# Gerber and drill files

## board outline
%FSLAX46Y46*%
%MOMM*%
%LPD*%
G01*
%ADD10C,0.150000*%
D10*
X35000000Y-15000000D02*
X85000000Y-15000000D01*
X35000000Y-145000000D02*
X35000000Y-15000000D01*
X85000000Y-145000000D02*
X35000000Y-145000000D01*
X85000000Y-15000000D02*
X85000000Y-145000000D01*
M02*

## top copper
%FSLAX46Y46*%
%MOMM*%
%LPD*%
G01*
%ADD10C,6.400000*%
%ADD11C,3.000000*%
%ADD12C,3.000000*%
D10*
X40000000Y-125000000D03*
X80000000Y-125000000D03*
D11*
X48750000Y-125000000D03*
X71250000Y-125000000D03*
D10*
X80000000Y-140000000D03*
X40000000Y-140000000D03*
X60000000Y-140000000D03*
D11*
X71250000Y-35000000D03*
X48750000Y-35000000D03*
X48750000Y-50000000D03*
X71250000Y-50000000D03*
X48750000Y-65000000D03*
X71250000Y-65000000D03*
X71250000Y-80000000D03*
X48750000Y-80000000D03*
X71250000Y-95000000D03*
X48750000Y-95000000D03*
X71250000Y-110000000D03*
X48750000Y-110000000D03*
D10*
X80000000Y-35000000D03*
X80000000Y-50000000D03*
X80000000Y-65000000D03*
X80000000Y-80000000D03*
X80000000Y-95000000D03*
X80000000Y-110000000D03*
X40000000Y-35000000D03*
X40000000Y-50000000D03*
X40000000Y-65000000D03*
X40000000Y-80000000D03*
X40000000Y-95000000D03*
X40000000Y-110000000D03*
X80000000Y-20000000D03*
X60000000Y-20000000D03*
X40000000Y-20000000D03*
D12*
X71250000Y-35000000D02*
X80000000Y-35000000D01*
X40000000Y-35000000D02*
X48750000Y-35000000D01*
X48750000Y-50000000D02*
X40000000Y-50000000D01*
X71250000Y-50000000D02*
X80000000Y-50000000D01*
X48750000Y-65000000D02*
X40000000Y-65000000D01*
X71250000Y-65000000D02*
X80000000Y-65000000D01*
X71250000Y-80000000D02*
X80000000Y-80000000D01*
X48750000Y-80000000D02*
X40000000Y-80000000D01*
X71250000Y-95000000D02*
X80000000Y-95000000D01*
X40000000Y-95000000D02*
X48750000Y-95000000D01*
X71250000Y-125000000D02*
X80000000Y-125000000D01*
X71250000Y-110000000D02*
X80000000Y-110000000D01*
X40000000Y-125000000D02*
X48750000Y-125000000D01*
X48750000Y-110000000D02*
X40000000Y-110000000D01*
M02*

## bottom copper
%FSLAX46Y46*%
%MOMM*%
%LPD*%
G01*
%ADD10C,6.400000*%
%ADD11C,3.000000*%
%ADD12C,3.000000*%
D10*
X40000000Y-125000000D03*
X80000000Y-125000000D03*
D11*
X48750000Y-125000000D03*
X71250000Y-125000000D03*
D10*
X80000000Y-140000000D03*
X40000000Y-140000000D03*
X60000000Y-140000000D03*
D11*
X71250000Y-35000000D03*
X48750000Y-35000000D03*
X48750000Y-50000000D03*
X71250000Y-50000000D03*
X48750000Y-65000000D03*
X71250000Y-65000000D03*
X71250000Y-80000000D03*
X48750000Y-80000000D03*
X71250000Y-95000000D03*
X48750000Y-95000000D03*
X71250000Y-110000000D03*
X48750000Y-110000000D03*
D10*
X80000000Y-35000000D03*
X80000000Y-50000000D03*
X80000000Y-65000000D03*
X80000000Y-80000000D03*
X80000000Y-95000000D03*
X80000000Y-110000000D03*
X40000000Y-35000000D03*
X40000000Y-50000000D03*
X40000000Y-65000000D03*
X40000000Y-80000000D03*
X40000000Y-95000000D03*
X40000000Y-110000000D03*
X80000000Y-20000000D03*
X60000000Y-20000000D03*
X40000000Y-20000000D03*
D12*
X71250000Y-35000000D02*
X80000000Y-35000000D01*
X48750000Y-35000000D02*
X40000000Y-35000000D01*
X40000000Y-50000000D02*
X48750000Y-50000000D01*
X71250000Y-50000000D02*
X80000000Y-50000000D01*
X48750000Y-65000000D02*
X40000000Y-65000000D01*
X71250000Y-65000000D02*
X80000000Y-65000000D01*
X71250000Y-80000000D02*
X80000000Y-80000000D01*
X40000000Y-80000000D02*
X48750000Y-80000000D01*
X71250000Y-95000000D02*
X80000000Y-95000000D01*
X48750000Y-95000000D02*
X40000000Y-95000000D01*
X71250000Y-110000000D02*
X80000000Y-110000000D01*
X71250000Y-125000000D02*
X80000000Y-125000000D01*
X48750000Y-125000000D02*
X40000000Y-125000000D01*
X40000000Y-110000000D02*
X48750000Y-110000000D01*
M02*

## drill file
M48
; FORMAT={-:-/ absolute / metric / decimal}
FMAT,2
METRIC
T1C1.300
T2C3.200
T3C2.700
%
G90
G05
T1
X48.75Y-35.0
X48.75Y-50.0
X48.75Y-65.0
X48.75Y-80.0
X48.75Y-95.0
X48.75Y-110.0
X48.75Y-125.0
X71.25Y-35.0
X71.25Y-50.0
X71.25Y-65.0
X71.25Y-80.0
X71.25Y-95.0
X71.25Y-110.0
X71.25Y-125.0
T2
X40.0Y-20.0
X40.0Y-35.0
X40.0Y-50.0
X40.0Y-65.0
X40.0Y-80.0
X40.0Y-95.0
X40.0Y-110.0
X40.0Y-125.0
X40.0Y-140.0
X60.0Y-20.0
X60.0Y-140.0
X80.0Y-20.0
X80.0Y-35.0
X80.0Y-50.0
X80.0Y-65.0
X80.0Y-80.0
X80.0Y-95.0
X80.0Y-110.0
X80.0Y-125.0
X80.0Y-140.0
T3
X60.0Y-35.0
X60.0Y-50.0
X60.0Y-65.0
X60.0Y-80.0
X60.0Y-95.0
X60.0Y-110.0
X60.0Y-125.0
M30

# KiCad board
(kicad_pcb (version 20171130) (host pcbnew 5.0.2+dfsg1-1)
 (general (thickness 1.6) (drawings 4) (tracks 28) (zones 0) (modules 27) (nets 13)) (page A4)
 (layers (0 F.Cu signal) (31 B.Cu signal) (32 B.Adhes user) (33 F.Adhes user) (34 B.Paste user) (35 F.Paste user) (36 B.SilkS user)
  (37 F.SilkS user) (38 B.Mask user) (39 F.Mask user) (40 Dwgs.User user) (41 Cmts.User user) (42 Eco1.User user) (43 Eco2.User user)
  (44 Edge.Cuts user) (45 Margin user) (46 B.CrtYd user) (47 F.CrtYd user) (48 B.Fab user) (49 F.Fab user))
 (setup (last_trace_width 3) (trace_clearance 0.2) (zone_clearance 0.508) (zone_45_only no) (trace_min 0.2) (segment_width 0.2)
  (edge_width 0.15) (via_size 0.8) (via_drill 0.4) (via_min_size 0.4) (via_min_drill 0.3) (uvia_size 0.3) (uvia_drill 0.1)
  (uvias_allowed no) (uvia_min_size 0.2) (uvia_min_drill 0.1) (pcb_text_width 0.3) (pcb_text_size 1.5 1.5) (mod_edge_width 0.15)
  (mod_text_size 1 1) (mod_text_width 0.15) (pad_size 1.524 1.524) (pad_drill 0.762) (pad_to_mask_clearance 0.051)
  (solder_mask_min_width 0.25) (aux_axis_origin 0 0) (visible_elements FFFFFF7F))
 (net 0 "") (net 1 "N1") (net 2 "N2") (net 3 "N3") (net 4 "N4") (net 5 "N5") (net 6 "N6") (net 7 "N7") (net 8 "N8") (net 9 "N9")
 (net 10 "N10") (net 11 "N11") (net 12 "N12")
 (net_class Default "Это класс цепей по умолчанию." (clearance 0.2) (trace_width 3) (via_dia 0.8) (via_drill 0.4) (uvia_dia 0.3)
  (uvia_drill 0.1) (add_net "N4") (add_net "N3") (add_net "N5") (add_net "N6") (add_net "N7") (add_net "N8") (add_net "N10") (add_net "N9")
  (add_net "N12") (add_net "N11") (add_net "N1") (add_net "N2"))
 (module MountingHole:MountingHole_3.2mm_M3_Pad (layer F.Cu) (at 40 125)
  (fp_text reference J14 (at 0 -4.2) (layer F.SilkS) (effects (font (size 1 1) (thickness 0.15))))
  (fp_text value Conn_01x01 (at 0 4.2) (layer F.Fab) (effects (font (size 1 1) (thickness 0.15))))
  (pad 1 thru_hole circle (at 0 0) (size 6.4 6.4) (drill 3.2) (layers *.Cu *.Mask) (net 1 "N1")))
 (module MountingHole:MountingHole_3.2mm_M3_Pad (layer F.Cu) (at 80 125)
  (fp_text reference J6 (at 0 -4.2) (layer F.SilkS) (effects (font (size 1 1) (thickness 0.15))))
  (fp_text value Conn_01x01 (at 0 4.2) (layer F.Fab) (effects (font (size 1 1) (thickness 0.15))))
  (pad 1 thru_hole circle (at 0 0) (size 6.4 6.4) (drill 3.2) (layers *.Cu *.Mask) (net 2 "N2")))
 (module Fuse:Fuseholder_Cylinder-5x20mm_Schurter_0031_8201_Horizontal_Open (layer F.Cu) (at 48.75 125)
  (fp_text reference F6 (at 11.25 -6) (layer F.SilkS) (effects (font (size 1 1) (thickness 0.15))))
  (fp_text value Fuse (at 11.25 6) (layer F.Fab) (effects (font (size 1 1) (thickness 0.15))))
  (pad 1 thru_hole circle (at 0 0) (size 3 3) (drill 1.3) (layers *.Cu *.Mask) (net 1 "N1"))
  (pad 2 thru_hole circle (at 22.5 0) (size 3 3) (drill 1.3) (layers *.Cu *.Mask) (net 2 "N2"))
  (pad "" np_thru_hole circle (at 11.25 0) (size 2.7 2.7) (drill 2.7) (layers *.Cu *.Mask)))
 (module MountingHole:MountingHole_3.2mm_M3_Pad (layer F.Cu) (at 80 140)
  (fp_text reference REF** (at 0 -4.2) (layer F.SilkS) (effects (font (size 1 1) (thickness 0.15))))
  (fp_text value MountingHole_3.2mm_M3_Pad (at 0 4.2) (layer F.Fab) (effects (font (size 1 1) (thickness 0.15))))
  (pad 1 thru_hole circle (at 0 0) (size 6.4 6.4) (drill 3.2) (layers *.Cu *.Mask)))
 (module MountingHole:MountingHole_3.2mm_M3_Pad (layer F.Cu) (at 40 140)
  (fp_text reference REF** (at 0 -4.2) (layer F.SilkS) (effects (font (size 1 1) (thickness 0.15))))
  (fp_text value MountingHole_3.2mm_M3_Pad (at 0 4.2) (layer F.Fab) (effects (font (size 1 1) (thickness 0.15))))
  (pad 1 thru_hole circle (at 0 0) (size 6.4 6.4) (drill 3.2) (layers *.Cu *.Mask)))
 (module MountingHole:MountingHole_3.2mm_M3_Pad (layer F.Cu) (at 60 140)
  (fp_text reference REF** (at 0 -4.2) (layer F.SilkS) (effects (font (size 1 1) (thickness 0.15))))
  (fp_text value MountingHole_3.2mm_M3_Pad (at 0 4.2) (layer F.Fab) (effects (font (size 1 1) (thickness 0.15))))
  (pad 1 thru_hole circle (at 0 0) (size 6.4 6.4) (drill 3.2) (layers *.Cu *.Mask)))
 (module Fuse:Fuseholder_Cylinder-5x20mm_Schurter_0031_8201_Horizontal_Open (layer F.Cu) (at 48.75 35)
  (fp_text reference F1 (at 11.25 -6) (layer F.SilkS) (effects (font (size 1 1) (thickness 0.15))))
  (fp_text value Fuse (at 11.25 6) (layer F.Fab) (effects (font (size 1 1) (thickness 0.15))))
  (pad "" np_thru_hole circle (at 11.25 0) (size 2.7 2.7) (drill 2.7) (layers *.Cu *.Mask))
  (pad 2 thru_hole circle (at 22.5 0) (size 3 3) (drill 1.3) (layers *.Cu *.Mask) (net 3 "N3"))
  (pad 1 thru_hole circle (at 0 0) (size 3 3) (drill 1.3) (layers *.Cu *.Mask) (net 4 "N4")))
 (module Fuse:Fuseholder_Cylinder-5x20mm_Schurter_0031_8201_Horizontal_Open (layer F.Cu) (at 48.75 50)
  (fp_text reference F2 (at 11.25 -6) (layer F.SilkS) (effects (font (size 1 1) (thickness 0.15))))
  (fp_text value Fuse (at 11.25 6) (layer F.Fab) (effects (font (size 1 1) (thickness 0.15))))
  (pad 1 thru_hole circle (at 0 0) (size 3 3) (drill 1.3) (layers *.Cu *.Mask) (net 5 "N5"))
  (pad 2 thru_hole circle (at 22.5 0) (size 3 3) (drill 1.3) (layers *.Cu *.Mask) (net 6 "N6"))
  (pad "" np_thru_hole circle (at 11.25 0) (size 2.7 2.7) (drill 2.7) (layers *.Cu *.Mask)))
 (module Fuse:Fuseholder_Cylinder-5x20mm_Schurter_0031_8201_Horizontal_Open (layer F.Cu) (at 48.75 65)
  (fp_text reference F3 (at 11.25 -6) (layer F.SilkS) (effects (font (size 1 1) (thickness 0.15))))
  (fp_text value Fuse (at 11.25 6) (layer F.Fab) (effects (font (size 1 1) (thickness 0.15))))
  (pad 1 thru_hole circle (at 0 0) (size 3 3) (drill 1.3) (layers *.Cu *.Mask) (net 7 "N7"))
  (pad 2 thru_hole circle (at 22.5 0) (size 3 3) (drill 1.3) (layers *.Cu *.Mask) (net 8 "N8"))
  (pad "" np_thru_hole circle (at 11.25 0) (size 2.7 2.7) (drill 2.7) (layers *.Cu *.Mask)))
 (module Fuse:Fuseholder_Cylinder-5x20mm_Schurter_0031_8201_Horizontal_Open (layer F.Cu) (at 48.75 80)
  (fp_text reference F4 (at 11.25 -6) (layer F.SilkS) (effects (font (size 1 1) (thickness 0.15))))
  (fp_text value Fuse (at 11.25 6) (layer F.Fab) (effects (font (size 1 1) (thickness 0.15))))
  (pad "" np_thru_hole circle (at 11.25 0) (size 2.7 2.7) (drill 2.7) (layers *.Cu *.Mask))
  (pad 2 thru_hole circle (at 22.5 0) (size 3 3) (drill 1.3) (layers *.Cu *.Mask) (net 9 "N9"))
  (pad 1 thru_hole circle (at 0 0) (size 3 3) (drill 1.3) (layers *.Cu *.Mask) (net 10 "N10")))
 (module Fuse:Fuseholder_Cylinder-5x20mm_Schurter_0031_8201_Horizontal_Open (layer F.Cu) (at 48.75 95)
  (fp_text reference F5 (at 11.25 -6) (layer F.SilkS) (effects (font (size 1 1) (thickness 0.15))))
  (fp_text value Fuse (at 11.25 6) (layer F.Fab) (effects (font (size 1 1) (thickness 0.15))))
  (pad "" np_thru_hole circle (at 11.25 0) (size 2.7 2.7) (drill 2.7) (layers *.Cu *.Mask))
  (pad 2 thru_hole circle (at 22.5 0) (size 3 3) (drill 1.3) (layers *.Cu *.Mask) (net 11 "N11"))
  (pad 1 thru_hole circle (at 0 0) (size 3 3) (drill 1.3) (layers *.Cu *.Mask) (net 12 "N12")))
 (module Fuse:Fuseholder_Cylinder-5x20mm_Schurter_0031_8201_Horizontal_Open (layer F.Cu) (at 48.75 110)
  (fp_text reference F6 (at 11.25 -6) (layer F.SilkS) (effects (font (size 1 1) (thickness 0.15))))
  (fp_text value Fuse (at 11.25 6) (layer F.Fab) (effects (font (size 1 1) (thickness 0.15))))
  (pad "" np_thru_hole circle (at 11.25 0) (size 2.7 2.7) (drill 2.7) (layers *.Cu *.Mask))
  (pad 2 thru_hole circle (at 22.5 0) (size 3 3) (drill 1.3) (layers *.Cu *.Mask) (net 2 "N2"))
  (pad 1 thru_hole circle (at 0 0) (size 3 3) (drill 1.3) (layers *.Cu *.Mask) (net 1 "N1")))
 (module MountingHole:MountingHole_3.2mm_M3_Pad (layer F.Cu) (at 80 35)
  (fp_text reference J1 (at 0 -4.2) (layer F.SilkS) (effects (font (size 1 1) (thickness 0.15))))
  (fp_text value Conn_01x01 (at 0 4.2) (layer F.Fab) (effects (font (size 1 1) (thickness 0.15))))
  (pad 1 thru_hole circle (at 0 0) (size 6.4 6.4) (drill 3.2) (layers *.Cu *.Mask) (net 3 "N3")))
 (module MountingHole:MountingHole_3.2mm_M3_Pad (layer F.Cu) (at 80 50)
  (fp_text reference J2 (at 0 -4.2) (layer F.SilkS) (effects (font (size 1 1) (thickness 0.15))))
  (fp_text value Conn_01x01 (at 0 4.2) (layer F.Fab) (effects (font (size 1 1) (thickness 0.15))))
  (pad 1 thru_hole circle (at 0 0) (size 6.4 6.4) (drill 3.2) (layers *.Cu *.Mask) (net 6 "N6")))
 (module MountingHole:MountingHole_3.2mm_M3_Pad (layer F.Cu) (at 80 65)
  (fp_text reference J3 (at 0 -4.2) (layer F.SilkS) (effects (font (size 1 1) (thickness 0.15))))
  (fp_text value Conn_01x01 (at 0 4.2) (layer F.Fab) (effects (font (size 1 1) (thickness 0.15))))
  (pad 1 thru_hole circle (at 0 0) (size 6.4 6.4) (drill 3.2) (layers *.Cu *.Mask) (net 8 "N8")))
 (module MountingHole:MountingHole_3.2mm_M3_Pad (layer F.Cu) (at 80 80)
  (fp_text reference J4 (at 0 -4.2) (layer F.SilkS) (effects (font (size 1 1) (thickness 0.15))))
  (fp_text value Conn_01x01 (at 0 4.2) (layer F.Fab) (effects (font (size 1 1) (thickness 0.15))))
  (pad 1 thru_hole circle (at 0 0) (size 6.4 6.4) (drill 3.2) (layers *.Cu *.Mask) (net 9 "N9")))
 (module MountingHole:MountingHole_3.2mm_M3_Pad (layer F.Cu) (at 80 95)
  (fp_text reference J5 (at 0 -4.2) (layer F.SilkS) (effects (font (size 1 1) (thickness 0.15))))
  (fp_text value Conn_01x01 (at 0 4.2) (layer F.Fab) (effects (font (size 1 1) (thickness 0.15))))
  (pad 1 thru_hole circle (at 0 0) (size 6.4 6.4) (drill 3.2) (layers *.Cu *.Mask) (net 11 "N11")))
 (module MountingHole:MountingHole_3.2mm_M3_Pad (layer F.Cu) (at 80 110)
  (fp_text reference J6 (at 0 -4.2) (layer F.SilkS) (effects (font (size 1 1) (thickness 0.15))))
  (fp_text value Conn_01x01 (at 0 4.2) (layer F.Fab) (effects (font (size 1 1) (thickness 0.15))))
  (pad 1 thru_hole circle (at 0 0) (size 6.4 6.4) (drill 3.2) (layers *.Cu *.Mask) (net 2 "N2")))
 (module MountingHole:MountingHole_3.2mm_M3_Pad (layer F.Cu) (at 40 35)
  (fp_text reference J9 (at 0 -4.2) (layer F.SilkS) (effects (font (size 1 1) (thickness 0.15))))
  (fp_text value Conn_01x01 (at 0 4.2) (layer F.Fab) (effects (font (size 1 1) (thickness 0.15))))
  (pad 1 thru_hole circle (at 0 0) (size 6.4 6.4) (drill 3.2) (layers *.Cu *.Mask) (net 4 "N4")))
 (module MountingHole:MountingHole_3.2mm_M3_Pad (layer F.Cu) (at 40 50)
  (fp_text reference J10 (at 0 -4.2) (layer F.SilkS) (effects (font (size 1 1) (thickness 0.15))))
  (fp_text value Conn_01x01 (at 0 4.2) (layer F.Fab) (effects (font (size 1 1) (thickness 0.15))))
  (pad 1 thru_hole circle (at 0 0) (size 6.4 6.4) (drill 3.2) (layers *.Cu *.Mask) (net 5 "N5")))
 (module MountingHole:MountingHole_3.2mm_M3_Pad (layer F.Cu) (at 40 65)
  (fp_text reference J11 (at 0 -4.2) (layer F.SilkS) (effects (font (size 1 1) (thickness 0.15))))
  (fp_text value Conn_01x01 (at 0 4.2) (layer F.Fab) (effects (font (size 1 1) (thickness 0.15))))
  (pad 1 thru_hole circle (at 0 0) (size 6.4 6.4) (drill 3.2) (layers *.Cu *.Mask) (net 7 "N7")))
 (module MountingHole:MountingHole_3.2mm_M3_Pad (layer F.Cu) (at 40 80)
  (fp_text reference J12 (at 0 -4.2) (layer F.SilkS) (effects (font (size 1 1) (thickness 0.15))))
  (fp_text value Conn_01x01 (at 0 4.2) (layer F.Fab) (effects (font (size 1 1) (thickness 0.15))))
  (pad 1 thru_hole circle (at 0 0) (size 6.4 6.4) (drill 3.2) (layers *.Cu *.Mask) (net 10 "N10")))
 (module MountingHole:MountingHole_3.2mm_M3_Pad (layer F.Cu) (at 40 95)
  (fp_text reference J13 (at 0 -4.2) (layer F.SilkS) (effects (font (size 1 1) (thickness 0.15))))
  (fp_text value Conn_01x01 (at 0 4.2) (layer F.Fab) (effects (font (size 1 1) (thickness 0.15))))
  (pad 1 thru_hole circle (at 0 0) (size 6.4 6.4) (drill 3.2) (layers *.Cu *.Mask) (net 12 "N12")))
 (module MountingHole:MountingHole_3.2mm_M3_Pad (layer F.Cu) (at 40 110)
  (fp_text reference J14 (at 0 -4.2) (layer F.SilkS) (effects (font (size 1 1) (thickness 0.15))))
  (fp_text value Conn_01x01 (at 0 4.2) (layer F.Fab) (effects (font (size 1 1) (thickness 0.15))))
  (pad 1 thru_hole circle (at 0 0) (size 6.4 6.4) (drill 3.2) (layers *.Cu *.Mask) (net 1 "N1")))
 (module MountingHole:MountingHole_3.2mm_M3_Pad (layer F.Cu) (at 80 20)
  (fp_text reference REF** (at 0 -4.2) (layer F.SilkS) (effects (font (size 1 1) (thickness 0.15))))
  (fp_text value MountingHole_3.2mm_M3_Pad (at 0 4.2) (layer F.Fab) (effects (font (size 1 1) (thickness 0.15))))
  (pad 1 thru_hole circle (at 0 0) (size 6.4 6.4) (drill 3.2) (layers *.Cu *.Mask)))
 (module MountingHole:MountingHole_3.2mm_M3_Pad (layer F.Cu) (at 60 20)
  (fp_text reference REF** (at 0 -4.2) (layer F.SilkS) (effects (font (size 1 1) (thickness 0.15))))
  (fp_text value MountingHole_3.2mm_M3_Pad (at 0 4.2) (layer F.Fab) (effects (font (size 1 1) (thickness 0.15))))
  (pad 1 thru_hole circle (at 0 0) (size 6.4 6.4) (drill 3.2) (layers *.Cu *.Mask)))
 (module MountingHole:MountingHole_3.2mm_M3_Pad (layer F.Cu) (at 40 20)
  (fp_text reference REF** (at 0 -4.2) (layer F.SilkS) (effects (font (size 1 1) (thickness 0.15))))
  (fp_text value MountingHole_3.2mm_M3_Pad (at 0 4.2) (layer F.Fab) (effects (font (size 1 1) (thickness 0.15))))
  (pad 1 thru_hole circle (at 0 0) (size 6.4 6.4) (drill 3.2) (layers *.Cu *.Mask)))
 (gr_line (start 35 15) (end 85 15) (layer Edge.Cuts) (width 0.15))
 (gr_line (start 35 145) (end 35 15) (layer Edge.Cuts) (width 0.15))
 (gr_line (start 85 145) (end 35 145) (layer Edge.Cuts) (width 0.15))
 (gr_line (start 85 15) (end 85 145) (layer Edge.Cuts) (width 0.15))
 (segment (start 71.25 35) (end 80 35) (width 3) (layer B.Cu) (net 3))
 (segment (start 71.25 35) (end 80 35) (width 3) (layer F.Cu) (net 3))
 (segment (start 48.75 35) (end 40 35) (width 3) (layer B.Cu) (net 4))
 (segment (start 40 35) (end 48.75 35) (width 3) (layer F.Cu) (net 4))
 (segment (start 40 50) (end 48.75 50) (width 3) (layer B.Cu) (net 5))
 (segment (start 48.75 50) (end 40 50) (width 3) (layer F.Cu) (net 5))
 (segment (start 71.25 50) (end 80 50) (width 3) (layer B.Cu) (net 6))
 (segment (start 71.25 50) (end 80 50) (width 3) (layer F.Cu) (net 6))
 (segment (start 48.75 65) (end 40 65) (width 3) (layer B.Cu) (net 7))
 (segment (start 48.75 65) (end 40 65) (width 3) (layer F.Cu) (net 7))
 (segment (start 71.25 65) (end 80 65) (width 3) (layer B.Cu) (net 8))
 (segment (start 71.25 65) (end 80 65) (width 3) (layer F.Cu) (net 8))
 (segment (start 71.25 80) (end 80 80) (width 3) (layer F.Cu) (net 9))
 (segment (start 71.25 80) (end 80 80) (width 3) (layer B.Cu) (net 9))
 (segment (start 48.75 80) (end 40 80) (width 3) (layer F.Cu) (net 10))
 (segment (start 40 80) (end 48.75 80) (width 3) (layer B.Cu) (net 10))
 (segment (start 71.25 95) (end 80 95) (width 3) (layer F.Cu) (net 11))
 (segment (start 71.25 95) (end 80 95) (width 3) (layer B.Cu) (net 11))
 (segment (start 40 95) (end 48.75 95) (width 3) (layer F.Cu) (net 12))
 (segment (start 48.75 95) (end 40 95) (width 3) (layer B.Cu) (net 12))
 (segment (start 71.25 125) (end 80 125) (width 3) (layer F.Cu) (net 2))
 (segment (start 71.25 110) (end 80 110) (width 3) (layer F.Cu) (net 2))
 (segment (start 71.25 110) (end 80 110) (width 3) (layer B.Cu) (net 2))
 (segment (start 71.25 125) (end 80 125) (width 3) (layer B.Cu) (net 2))
 (segment (start 40 125) (end 48.75 125) (width 3) (layer F.Cu) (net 1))
 (segment (start 48.75 110) (end 40 110) (width 3) (layer F.Cu) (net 1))
 (segment (start 48.75 125) (end 40 125) (width 3) (layer B.Cu) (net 1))
 (segment (start 40 110) (end 48.75 110) (width 3) (layer B.Cu) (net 1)))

